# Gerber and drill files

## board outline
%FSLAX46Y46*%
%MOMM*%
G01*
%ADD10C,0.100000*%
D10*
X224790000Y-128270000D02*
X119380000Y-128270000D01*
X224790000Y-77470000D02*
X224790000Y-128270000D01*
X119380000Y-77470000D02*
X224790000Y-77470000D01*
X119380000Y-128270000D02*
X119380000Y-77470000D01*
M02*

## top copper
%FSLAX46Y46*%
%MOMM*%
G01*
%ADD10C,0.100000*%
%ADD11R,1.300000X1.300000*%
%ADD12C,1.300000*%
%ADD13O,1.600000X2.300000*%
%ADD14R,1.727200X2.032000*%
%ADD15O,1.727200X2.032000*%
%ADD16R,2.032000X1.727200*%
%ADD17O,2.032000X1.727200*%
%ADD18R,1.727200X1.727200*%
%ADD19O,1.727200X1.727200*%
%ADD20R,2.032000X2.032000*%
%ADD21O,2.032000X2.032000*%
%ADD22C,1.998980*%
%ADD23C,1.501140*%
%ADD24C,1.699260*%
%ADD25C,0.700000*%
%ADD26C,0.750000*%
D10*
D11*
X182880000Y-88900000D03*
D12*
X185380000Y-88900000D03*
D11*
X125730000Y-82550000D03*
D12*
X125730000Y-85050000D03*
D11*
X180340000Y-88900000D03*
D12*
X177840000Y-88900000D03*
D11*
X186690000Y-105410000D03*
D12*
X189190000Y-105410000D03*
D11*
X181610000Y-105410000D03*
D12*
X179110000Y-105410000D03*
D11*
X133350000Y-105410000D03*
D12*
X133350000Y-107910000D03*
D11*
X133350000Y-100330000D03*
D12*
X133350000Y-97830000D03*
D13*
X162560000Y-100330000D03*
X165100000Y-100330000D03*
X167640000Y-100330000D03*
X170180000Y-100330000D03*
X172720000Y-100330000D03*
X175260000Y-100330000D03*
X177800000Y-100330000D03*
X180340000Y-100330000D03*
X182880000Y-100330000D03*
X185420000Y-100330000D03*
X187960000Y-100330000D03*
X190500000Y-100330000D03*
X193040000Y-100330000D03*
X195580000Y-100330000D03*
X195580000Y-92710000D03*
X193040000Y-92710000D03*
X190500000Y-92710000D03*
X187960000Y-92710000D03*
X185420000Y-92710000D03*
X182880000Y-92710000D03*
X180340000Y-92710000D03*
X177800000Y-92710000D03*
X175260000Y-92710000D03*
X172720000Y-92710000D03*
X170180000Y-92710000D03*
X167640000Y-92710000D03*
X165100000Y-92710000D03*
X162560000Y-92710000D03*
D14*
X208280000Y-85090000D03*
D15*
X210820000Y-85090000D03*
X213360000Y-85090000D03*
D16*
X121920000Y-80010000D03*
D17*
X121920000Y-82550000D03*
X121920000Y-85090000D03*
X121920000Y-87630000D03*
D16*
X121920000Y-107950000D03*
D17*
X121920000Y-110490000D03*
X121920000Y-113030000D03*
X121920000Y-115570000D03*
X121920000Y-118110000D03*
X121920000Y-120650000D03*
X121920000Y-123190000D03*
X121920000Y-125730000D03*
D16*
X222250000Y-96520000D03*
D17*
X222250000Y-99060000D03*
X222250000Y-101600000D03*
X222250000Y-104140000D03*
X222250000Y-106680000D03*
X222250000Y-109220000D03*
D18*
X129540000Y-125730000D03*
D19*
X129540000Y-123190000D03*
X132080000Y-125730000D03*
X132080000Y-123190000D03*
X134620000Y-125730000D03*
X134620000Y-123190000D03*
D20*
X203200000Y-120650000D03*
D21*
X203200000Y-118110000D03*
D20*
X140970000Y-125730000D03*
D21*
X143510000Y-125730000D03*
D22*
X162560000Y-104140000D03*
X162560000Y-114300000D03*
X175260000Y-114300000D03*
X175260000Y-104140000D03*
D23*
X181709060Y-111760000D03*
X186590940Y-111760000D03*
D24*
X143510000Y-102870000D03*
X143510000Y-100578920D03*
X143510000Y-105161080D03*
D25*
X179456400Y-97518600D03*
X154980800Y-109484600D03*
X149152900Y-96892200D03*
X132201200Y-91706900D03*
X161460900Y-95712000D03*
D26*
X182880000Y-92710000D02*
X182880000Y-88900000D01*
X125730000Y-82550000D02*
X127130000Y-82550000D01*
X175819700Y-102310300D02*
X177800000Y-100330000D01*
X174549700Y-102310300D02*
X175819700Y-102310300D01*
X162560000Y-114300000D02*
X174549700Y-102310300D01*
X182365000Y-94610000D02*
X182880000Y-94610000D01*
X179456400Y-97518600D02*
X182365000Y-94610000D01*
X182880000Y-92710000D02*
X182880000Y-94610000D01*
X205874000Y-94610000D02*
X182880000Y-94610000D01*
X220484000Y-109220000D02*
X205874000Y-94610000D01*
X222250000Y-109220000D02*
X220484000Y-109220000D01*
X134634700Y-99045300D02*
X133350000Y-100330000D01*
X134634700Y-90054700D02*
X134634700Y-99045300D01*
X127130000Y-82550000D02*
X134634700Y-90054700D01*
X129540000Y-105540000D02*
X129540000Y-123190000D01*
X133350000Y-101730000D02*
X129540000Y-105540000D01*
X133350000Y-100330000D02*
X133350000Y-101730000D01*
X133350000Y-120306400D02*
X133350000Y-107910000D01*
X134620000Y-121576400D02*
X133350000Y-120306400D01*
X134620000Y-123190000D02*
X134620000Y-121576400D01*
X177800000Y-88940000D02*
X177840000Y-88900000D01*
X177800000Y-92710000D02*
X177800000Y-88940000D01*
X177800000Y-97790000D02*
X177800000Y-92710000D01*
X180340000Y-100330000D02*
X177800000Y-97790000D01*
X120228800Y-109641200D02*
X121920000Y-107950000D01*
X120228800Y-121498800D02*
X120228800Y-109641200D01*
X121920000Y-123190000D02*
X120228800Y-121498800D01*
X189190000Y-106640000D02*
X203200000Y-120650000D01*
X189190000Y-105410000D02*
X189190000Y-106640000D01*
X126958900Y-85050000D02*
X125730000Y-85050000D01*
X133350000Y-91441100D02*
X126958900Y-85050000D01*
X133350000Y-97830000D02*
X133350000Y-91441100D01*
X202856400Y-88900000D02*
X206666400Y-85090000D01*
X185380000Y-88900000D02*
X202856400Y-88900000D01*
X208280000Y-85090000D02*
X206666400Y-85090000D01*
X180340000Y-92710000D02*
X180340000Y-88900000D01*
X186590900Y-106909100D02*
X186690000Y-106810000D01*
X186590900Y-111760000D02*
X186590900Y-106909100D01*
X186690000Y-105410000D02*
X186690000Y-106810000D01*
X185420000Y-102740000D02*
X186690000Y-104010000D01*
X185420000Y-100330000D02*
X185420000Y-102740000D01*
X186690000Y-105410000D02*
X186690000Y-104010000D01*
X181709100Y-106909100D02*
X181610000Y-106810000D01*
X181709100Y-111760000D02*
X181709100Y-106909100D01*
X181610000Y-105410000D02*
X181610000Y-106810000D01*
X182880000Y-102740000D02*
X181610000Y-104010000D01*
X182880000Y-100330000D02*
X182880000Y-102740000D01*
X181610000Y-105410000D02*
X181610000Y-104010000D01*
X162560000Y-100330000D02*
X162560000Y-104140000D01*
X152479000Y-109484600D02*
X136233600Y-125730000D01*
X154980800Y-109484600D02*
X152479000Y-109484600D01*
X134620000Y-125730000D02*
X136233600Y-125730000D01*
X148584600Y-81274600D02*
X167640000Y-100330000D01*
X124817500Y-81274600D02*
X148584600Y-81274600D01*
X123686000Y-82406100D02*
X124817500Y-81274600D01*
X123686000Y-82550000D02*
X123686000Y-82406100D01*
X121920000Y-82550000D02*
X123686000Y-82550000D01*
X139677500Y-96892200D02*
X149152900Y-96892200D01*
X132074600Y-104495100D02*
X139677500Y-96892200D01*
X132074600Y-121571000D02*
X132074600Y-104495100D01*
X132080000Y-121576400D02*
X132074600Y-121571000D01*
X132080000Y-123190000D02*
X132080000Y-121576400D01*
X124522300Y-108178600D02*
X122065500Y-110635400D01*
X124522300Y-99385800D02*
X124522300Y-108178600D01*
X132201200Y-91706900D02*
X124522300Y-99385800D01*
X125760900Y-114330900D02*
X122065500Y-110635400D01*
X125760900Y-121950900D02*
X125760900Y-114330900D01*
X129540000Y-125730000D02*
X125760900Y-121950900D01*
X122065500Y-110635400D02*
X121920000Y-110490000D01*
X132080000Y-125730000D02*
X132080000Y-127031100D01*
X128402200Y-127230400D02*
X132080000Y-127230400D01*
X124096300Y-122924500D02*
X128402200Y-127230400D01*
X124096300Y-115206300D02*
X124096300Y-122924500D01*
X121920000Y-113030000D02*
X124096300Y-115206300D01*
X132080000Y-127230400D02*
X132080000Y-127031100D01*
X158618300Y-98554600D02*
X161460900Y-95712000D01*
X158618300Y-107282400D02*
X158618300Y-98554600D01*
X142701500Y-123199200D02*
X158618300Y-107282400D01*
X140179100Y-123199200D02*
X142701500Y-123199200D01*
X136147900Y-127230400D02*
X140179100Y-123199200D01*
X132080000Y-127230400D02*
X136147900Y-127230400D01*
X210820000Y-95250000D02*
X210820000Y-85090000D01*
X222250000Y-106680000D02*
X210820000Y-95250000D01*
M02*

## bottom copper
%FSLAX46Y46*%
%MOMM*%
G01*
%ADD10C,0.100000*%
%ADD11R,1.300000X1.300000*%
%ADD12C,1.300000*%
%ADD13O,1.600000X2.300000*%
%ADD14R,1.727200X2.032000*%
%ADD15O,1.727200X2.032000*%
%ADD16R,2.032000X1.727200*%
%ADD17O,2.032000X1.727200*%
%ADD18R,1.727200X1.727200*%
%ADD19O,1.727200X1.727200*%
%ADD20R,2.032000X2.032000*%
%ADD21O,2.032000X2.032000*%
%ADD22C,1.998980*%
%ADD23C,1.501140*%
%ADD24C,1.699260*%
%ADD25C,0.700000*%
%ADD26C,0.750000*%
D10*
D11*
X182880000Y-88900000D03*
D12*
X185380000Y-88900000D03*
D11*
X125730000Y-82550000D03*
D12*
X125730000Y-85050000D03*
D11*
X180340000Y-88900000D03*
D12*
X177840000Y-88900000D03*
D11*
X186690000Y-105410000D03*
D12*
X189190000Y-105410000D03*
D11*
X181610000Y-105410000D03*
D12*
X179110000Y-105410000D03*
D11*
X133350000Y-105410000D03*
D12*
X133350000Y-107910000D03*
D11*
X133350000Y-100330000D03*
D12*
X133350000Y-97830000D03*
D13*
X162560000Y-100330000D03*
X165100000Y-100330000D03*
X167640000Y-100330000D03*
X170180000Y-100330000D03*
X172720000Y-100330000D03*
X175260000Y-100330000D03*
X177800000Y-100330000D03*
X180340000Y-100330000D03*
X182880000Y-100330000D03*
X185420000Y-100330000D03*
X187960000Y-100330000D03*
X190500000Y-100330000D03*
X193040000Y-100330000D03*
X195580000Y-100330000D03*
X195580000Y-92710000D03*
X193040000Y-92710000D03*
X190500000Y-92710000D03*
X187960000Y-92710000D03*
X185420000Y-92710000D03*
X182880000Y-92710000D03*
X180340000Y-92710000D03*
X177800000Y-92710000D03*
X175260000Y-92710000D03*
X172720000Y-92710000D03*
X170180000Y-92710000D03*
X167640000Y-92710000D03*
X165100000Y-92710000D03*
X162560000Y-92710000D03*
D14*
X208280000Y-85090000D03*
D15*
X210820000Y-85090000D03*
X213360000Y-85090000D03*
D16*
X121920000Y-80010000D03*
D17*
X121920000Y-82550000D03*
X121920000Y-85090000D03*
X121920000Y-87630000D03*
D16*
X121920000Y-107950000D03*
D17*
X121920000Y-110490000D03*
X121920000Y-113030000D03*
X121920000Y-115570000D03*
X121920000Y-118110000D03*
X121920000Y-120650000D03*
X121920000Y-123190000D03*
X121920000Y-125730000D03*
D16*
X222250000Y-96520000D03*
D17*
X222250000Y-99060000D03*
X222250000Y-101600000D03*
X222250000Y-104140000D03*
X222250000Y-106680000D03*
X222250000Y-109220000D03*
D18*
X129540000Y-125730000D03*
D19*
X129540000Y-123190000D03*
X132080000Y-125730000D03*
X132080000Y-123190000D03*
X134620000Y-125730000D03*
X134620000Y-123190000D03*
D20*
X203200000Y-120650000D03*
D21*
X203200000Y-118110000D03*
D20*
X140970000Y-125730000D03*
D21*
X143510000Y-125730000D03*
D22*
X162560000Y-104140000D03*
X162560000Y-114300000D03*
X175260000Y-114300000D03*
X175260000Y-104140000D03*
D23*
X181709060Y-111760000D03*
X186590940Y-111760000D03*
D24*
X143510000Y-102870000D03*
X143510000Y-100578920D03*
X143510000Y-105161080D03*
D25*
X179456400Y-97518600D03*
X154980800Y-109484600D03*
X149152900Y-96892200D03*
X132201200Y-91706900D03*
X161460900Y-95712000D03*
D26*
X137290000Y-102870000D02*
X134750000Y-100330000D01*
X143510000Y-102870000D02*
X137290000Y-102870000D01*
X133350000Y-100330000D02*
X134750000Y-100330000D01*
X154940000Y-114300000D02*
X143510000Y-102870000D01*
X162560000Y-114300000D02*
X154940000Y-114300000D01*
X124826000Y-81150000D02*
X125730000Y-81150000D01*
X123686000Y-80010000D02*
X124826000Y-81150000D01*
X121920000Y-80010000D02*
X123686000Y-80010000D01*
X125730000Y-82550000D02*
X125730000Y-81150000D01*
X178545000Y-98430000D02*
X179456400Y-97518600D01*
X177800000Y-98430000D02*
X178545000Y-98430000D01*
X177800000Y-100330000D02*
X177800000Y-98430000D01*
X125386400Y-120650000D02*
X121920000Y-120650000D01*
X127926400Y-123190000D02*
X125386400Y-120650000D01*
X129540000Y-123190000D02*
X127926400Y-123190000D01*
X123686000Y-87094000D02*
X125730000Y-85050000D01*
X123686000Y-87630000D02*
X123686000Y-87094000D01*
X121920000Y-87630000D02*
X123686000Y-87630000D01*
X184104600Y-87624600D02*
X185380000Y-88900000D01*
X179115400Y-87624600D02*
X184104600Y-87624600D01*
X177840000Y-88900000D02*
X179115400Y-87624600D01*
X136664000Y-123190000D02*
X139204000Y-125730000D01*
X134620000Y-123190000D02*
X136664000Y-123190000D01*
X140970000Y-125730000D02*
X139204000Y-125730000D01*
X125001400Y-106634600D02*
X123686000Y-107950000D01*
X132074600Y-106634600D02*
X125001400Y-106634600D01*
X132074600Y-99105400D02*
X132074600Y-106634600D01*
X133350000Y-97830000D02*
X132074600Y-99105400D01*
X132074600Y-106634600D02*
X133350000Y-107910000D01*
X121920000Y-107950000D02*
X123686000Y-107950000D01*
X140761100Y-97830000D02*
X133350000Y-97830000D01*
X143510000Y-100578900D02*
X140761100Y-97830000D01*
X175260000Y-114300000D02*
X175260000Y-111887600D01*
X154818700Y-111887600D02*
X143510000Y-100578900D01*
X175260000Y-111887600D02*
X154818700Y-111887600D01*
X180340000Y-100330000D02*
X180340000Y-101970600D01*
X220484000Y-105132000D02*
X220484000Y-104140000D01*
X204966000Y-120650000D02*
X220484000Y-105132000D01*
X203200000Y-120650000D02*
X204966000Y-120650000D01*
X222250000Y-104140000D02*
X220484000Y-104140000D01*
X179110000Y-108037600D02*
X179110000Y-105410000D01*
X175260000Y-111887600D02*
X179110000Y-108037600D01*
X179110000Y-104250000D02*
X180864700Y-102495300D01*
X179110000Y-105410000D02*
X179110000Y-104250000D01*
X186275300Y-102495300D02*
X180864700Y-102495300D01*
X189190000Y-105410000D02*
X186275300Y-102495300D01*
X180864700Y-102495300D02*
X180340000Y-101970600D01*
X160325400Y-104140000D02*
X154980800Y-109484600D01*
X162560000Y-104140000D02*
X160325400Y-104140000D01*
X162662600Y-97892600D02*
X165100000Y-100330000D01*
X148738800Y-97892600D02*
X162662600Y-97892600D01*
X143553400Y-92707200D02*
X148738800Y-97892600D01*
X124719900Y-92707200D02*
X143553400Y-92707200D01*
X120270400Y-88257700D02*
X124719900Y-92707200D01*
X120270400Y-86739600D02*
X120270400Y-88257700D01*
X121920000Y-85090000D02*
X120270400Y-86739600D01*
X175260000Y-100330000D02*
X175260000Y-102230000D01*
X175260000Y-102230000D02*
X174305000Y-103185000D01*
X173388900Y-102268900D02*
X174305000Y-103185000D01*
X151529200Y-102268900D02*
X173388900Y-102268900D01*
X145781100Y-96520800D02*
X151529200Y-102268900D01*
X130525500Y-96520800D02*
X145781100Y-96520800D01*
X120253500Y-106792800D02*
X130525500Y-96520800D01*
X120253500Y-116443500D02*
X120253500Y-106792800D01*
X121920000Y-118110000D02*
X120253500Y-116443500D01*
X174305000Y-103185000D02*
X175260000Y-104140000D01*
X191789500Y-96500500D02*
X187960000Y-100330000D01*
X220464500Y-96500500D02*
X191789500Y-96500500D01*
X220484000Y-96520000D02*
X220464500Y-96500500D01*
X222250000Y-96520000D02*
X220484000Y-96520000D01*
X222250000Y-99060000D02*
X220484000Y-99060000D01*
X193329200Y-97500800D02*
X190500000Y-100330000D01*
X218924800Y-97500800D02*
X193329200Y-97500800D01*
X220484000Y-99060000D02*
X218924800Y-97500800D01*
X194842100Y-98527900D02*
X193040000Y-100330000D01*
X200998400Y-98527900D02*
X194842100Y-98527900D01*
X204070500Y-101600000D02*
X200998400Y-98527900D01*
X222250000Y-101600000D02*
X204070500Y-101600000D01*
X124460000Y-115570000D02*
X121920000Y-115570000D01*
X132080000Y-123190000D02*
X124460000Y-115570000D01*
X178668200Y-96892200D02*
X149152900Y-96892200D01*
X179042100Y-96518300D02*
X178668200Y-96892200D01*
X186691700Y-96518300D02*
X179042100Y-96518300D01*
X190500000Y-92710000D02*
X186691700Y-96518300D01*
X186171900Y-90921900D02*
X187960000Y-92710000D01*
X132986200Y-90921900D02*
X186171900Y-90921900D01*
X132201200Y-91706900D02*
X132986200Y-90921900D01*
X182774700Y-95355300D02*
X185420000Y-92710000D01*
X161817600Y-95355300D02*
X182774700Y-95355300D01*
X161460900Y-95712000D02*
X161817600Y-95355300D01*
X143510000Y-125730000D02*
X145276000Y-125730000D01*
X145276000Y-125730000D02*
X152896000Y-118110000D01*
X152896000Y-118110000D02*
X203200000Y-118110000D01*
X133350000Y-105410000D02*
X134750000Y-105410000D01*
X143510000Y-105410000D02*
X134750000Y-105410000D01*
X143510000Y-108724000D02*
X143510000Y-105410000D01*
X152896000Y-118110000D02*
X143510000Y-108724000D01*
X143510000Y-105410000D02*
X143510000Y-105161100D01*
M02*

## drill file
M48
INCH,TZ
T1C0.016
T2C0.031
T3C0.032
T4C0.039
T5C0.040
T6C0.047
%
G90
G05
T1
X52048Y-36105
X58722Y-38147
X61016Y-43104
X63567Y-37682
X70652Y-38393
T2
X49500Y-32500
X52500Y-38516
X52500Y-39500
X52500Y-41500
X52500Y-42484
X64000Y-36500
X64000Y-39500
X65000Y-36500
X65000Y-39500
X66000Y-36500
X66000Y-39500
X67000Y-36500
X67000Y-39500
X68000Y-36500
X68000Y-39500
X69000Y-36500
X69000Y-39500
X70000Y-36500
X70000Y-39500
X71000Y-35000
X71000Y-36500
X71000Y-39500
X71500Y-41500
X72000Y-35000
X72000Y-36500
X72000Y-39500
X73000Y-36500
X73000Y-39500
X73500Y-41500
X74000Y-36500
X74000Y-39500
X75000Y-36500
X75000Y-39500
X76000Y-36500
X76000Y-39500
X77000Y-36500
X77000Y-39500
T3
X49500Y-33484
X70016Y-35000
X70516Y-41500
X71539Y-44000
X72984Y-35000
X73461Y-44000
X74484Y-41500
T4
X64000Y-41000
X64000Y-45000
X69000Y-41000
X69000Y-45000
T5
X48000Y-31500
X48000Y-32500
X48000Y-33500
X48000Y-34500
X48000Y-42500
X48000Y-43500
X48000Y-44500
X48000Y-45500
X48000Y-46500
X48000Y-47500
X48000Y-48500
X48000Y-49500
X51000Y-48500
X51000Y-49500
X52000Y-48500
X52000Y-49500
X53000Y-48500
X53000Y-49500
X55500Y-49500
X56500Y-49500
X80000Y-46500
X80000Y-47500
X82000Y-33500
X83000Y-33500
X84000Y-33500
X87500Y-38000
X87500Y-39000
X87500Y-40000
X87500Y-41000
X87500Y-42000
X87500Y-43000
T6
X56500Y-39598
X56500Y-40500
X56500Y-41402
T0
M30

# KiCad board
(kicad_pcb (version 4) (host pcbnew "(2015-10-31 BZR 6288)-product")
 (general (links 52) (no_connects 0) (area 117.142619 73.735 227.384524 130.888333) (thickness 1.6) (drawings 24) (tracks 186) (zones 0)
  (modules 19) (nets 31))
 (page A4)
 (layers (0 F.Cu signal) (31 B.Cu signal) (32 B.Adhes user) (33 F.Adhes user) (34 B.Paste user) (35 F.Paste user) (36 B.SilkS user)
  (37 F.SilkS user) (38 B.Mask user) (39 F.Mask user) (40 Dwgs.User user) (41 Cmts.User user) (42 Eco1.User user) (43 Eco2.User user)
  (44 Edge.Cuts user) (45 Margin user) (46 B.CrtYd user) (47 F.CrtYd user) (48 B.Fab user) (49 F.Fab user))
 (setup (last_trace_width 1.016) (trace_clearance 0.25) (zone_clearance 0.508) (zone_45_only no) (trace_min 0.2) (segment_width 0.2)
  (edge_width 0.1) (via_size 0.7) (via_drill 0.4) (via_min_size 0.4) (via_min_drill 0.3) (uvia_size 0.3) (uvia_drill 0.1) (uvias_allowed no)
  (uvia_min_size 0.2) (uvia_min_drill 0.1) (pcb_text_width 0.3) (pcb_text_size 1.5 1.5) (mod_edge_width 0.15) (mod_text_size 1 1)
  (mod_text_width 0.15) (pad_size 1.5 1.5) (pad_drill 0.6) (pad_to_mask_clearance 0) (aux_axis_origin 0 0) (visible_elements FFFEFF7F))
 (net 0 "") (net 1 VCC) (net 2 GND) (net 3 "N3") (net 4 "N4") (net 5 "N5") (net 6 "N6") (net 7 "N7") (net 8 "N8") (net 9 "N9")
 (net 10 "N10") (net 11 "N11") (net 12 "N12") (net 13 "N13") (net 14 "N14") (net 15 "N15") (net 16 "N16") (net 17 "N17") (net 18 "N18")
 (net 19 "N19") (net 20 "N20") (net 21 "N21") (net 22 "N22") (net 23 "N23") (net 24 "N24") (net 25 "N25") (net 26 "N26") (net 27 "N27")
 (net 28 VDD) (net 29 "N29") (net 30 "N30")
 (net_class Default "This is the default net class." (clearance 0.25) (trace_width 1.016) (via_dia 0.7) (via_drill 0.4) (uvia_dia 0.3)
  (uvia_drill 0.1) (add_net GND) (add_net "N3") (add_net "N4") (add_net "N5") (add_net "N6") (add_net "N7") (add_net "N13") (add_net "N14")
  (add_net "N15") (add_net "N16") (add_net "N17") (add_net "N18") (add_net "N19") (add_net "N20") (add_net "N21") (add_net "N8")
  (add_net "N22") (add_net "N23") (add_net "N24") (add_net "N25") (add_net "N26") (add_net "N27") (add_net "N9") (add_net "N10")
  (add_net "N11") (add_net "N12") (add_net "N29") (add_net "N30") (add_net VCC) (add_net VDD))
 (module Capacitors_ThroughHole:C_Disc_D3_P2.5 (layer F.Cu) (at 182.88 88.9)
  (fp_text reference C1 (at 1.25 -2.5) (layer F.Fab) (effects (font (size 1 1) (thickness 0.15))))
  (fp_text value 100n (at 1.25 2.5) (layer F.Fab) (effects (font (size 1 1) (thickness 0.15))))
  (pad 1 thru_hole rect (at 0 0) (size 1.3 1.3) (drill 0.8) (layers *.Cu *.Mask F.SilkS) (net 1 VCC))
  (pad 2 thru_hole circle (at 2.5 0) (size 1.3 1.3) (drill 0.8001) (layers *.Cu *.Mask F.SilkS) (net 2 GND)))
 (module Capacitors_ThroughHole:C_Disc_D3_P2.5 (layer F.Cu) (at 125.73 82.55 270)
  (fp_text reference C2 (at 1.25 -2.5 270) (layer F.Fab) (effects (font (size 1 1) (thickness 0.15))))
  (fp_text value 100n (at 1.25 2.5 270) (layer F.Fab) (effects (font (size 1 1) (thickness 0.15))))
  (pad 1 thru_hole rect (at 0 0 270) (size 1.3 1.3) (drill 0.8) (layers *.Cu *.Mask F.SilkS) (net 1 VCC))
  (pad 2 thru_hole circle (at 2.5 0 270) (size 1.3 1.3) (drill 0.8001) (layers *.Cu *.Mask F.SilkS) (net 2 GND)))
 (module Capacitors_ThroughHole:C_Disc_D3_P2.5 (layer F.Cu) (at 180.34 88.9 180)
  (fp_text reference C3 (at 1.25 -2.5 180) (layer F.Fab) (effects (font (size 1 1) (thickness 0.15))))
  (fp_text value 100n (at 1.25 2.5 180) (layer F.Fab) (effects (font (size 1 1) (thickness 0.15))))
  (pad 1 thru_hole rect (at 0 0 180) (size 1.3 1.3) (drill 0.8) (layers *.Cu *.Mask F.SilkS) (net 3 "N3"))
  (pad 2 thru_hole circle (at 2.5 0 180) (size 1.3 1.3) (drill 0.8001) (layers *.Cu *.Mask F.SilkS) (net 2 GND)))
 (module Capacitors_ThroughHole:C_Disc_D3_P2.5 (layer F.Cu) (at 186.69 105.41)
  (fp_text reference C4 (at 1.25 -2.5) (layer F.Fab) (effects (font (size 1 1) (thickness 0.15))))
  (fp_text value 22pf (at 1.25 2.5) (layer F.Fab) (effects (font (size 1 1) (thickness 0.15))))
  (pad 1 thru_hole rect (at 0 0) (size 1.3 1.3) (drill 0.8) (layers *.Cu *.Mask F.SilkS) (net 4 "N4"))
  (pad 2 thru_hole circle (at 2.5 0) (size 1.3 1.3) (drill 0.8001) (layers *.Cu *.Mask F.SilkS) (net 2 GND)))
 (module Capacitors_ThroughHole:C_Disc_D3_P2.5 (layer F.Cu) (at 181.61 105.41 180)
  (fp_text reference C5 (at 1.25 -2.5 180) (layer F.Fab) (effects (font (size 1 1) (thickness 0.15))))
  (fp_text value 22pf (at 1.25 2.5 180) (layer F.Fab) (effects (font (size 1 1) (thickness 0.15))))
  (pad 1 thru_hole rect (at 0 0 180) (size 1.3 1.3) (drill 0.8) (layers *.Cu *.Mask F.SilkS) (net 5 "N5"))
  (pad 2 thru_hole circle (at 2.5 0 180) (size 1.3 1.3) (drill 0.8001) (layers *.Cu *.Mask F.SilkS) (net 2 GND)))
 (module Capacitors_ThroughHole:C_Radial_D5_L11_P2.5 (layer F.Cu) (at 133.35 105.41 270)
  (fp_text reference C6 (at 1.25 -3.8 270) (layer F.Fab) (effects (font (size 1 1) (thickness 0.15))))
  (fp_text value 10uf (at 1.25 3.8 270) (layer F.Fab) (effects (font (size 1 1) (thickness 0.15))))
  (pad 1 thru_hole rect (at 0 0 270) (size 1.3 1.3) (drill 0.8) (layers *.Cu *.Mask F.SilkS) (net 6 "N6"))
  (pad 2 thru_hole circle (at 2.5 0 270) (size 1.3 1.3) (drill 0.8) (layers *.Cu *.Mask F.SilkS) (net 2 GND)))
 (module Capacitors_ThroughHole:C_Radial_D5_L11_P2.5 (layer F.Cu) (at 133.35 100.33 90)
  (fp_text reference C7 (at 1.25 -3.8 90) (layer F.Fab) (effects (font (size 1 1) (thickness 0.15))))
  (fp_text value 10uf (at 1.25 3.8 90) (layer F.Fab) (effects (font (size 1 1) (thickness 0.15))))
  (pad 1 thru_hole rect (at 0 0 90) (size 1.3 1.3) (drill 0.8) (layers *.Cu *.Mask F.SilkS) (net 1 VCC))
  (pad 2 thru_hole circle (at 2.5 0 90) (size 1.3 1.3) (drill 0.8) (layers *.Cu *.Mask F.SilkS) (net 2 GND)))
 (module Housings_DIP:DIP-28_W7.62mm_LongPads (layer F.Cu) (at 162.56 100.33 90)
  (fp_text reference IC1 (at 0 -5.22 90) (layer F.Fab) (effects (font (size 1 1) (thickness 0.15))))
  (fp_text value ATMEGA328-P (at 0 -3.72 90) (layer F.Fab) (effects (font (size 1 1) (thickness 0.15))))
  (pad 1 thru_hole oval (at 0 0 90) (size 2.3 1.6) (drill 0.8) (layers *.Cu *.Mask F.SilkS) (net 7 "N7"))
  (pad 2 thru_hole oval (at 0 2.54 90) (size 2.3 1.6) (drill 0.8) (layers *.Cu *.Mask F.SilkS) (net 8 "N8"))
  (pad 3 thru_hole oval (at 0 5.08 90) (size 2.3 1.6) (drill 0.8) (layers *.Cu *.Mask F.SilkS) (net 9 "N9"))
  (pad 4 thru_hole oval (at 0 7.62 90) (size 2.3 1.6) (drill 0.8) (layers *.Cu *.Mask F.SilkS) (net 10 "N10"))
  (pad 5 thru_hole oval (at 0 10.16 90) (size 2.3 1.6) (drill 0.8) (layers *.Cu *.Mask F.SilkS) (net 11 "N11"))
  (pad 6 thru_hole oval (at 0 12.7 90) (size 2.3 1.6) (drill 0.8) (layers *.Cu *.Mask F.SilkS) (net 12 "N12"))
  (pad 7 thru_hole oval (at 0 15.24 90) (size 2.3 1.6) (drill 0.8) (layers *.Cu *.Mask F.SilkS) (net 1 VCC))
  (pad 8 thru_hole oval (at 0 17.78 90) (size 2.3 1.6) (drill 0.8) (layers *.Cu *.Mask F.SilkS) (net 2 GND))
  (pad 9 thru_hole oval (at 0 20.32 90) (size 2.3 1.6) (drill 0.8) (layers *.Cu *.Mask F.SilkS) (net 5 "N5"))
  (pad 10 thru_hole oval (at 0 22.86 90) (size 2.3 1.6) (drill 0.8) (layers *.Cu *.Mask F.SilkS) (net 4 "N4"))
  (pad 11 thru_hole oval (at 0 25.4 90) (size 2.3 1.6) (drill 0.8) (layers *.Cu *.Mask F.SilkS) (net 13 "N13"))
  (pad 12 thru_hole oval (at 0 27.94 90) (size 2.3 1.6) (drill 0.8) (layers *.Cu *.Mask F.SilkS) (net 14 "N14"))
  (pad 13 thru_hole oval (at 0 30.48 90) (size 2.3 1.6) (drill 0.8) (layers *.Cu *.Mask F.SilkS) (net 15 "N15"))
  (pad 14 thru_hole oval (at 0 33.02 90) (size 2.3 1.6) (drill 0.8) (layers *.Cu *.Mask F.SilkS) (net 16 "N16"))
  (pad 15 thru_hole oval (at 7.62 33.02 90) (size 2.3 1.6) (drill 0.8) (layers *.Cu *.Mask F.SilkS) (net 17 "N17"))
  (pad 16 thru_hole oval (at 7.62 30.48 90) (size 2.3 1.6) (drill 0.8) (layers *.Cu *.Mask F.SilkS) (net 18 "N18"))
  (pad 17 thru_hole oval (at 7.62 27.94 90) (size 2.3 1.6) (drill 0.8) (layers *.Cu *.Mask F.SilkS) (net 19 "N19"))
  (pad 18 thru_hole oval (at 7.62 25.4 90) (size 2.3 1.6) (drill 0.8) (layers *.Cu *.Mask F.SilkS) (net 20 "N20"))
  (pad 19 thru_hole oval (at 7.62 22.86 90) (size 2.3 1.6) (drill 0.8) (layers *.Cu *.Mask F.SilkS) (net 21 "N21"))
  (pad 20 thru_hole oval (at 7.62 20.32 90) (size 2.3 1.6) (drill 0.8) (layers *.Cu *.Mask F.SilkS) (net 1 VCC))
  (pad 21 thru_hole oval (at 7.62 17.78 90) (size 2.3 1.6) (drill 0.8) (layers *.Cu *.Mask F.SilkS) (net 3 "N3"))
  (pad 22 thru_hole oval (at 7.62 15.24 90) (size 2.3 1.6) (drill 0.8) (layers *.Cu *.Mask F.SilkS) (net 2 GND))
  (pad 23 thru_hole oval (at 7.62 12.7 90) (size 2.3 1.6) (drill 0.8) (layers *.Cu *.Mask F.SilkS) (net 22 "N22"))
  (pad 24 thru_hole oval (at 7.62 10.16 90) (size 2.3 1.6) (drill 0.8) (layers *.Cu *.Mask F.SilkS) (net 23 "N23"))
  (pad 25 thru_hole oval (at 7.62 7.62 90) (size 2.3 1.6) (drill 0.8) (layers *.Cu *.Mask F.SilkS) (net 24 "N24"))
  (pad 26 thru_hole oval (at 7.62 5.08 90) (size 2.3 1.6) (drill 0.8) (layers *.Cu *.Mask F.SilkS) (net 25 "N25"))
  (pad 27 thru_hole oval (at 7.62 2.54 90) (size 2.3 1.6) (drill 0.8) (layers *.Cu *.Mask F.SilkS) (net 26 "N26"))
  (pad 28 thru_hole oval (at 7.62 0 90) (size 2.3 1.6) (drill 0.8) (layers *.Cu *.Mask F.SilkS) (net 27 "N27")))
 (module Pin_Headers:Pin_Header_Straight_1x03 (layer F.Cu) (at 208.28 85.09 90)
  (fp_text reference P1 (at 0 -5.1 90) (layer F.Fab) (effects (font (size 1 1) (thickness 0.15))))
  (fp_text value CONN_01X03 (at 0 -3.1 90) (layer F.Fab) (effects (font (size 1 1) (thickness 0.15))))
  (pad 1 thru_hole rect (at 0 0 90) (size 2.032 1.7272) (drill 1.016) (layers *.Cu *.Mask F.SilkS) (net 2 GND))
  (pad 2 thru_hole oval (at 0 2.54 90) (size 2.032 1.7272) (drill 1.016) (layers *.Cu *.Mask F.SilkS) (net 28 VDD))
  (pad 3 thru_hole oval (at 0 5.08 90) (size 2.032 1.7272) (drill 1.016) (layers *.Cu *.Mask F.SilkS) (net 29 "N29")))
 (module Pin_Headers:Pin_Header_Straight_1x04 (layer F.Cu) (at 121.92 80.01)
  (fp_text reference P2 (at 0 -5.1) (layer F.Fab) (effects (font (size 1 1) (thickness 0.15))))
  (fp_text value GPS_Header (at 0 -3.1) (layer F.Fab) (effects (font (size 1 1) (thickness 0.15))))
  (pad 1 thru_hole rect (at 0 0) (size 2.032 1.7272) (drill 1.016) (layers *.Cu *.Mask F.SilkS) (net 1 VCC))
  (pad 2 thru_hole oval (at 0 2.54) (size 2.032 1.7272) (drill 1.016) (layers *.Cu *.Mask F.SilkS) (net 9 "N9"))
  (pad 3 thru_hole oval (at 0 5.08) (size 2.032 1.7272) (drill 1.016) (layers *.Cu *.Mask F.SilkS) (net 8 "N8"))
  (pad 4 thru_hole oval (at 0 7.62) (size 2.032 1.7272) (drill 1.016) (layers *.Cu *.Mask F.SilkS) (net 2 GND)))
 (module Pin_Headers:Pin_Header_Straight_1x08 (layer F.Cu) (at 121.92 107.95)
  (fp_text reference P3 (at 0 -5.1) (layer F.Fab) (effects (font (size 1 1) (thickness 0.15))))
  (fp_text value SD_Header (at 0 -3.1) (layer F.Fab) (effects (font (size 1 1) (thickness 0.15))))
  (pad 1 thru_hole rect (at 0 0) (size 2.032 1.7272) (drill 1.016) (layers *.Cu *.Mask F.SilkS) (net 2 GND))
  (pad 2 thru_hole oval (at 0 2.54) (size 2.032 1.7272) (drill 1.016) (layers *.Cu *.Mask F.SilkS) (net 20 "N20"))
  (pad 3 thru_hole oval (at 0 5.08) (size 2.032 1.7272) (drill 1.016) (layers *.Cu *.Mask F.SilkS) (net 21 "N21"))
  (pad 4 thru_hole oval (at 0 7.62) (size 2.032 1.7272) (drill 1.016) (layers *.Cu *.Mask F.SilkS) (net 19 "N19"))
  (pad 5 thru_hole oval (at 0 10.16) (size 2.032 1.7272) (drill 1.016) (layers *.Cu *.Mask F.SilkS) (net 12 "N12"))
  (pad 6 thru_hole oval (at 0 12.7) (size 2.032 1.7272) (drill 1.016) (layers *.Cu *.Mask F.SilkS) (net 1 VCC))
  (pad 7 thru_hole oval (at 0 15.24) (size 2.032 1.7272) (drill 1.016) (layers *.Cu *.Mask F.SilkS) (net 2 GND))
  (pad 8 thru_hole oval (at 0 17.78) (size 2.032 1.7272) (drill 1.016) (layers *.Cu *.Mask F.SilkS) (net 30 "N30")))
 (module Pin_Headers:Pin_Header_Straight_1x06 (layer F.Cu) (at 222.25 96.52)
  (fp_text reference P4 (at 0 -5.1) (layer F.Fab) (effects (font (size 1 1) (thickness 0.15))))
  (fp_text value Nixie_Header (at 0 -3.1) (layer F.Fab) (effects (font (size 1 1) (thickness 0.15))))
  (pad 1 thru_hole rect (at 0 0) (size 2.032 1.7272) (drill 1.016) (layers *.Cu *.Mask F.SilkS) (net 13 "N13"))
  (pad 2 thru_hole oval (at 0 2.54) (size 2.032 1.7272) (drill 1.016) (layers *.Cu *.Mask F.SilkS) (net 14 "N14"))
  (pad 3 thru_hole oval (at 0 5.08) (size 2.032 1.7272) (drill 1.016) (layers *.Cu *.Mask F.SilkS) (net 15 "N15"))
  (pad 4 thru_hole oval (at 0 7.62) (size 2.032 1.7272) (drill 1.016) (layers *.Cu *.Mask F.SilkS) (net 2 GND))
  (pad 5 thru_hole oval (at 0 10.16) (size 2.032 1.7272) (drill 1.016) (layers *.Cu *.Mask F.SilkS) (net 28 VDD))
  (pad 6 thru_hole oval (at 0 12.7) (size 2.032 1.7272) (drill 1.016) (layers *.Cu *.Mask F.SilkS) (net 1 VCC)))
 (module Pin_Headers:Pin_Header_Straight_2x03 (layer F.Cu) (at 129.54 125.73 90)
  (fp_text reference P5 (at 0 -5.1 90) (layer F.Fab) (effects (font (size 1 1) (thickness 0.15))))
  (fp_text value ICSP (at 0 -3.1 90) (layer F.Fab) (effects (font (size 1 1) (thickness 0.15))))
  (pad 1 thru_hole rect (at 0 0 90) (size 1.7272 1.7272) (drill 1.016) (layers *.Cu *.Mask F.SilkS) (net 20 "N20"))
  (pad 2 thru_hole oval (at 2.54 0 90) (size 1.7272 1.7272) (drill 1.016) (layers *.Cu *.Mask F.SilkS) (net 1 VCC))
  (pad 3 thru_hole oval (at 0 2.54 90) (size 1.7272 1.7272) (drill 1.016) (layers *.Cu *.Mask F.SilkS) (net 21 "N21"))
  (pad 4 thru_hole oval (at 2.54 2.54 90) (size 1.7272 1.7272) (drill 1.016) (layers *.Cu *.Mask F.SilkS) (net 19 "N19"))
  (pad 5 thru_hole oval (at 0 5.08 90) (size 1.7272 1.7272) (drill 1.016) (layers *.Cu *.Mask F.SilkS) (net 7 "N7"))
  (pad 6 thru_hole oval (at 2.54 5.08 90) (size 1.7272 1.7272) (drill 1.016) (layers *.Cu *.Mask F.SilkS) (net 2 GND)))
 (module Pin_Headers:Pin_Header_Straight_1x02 (layer F.Cu) (at 203.2 120.65 180)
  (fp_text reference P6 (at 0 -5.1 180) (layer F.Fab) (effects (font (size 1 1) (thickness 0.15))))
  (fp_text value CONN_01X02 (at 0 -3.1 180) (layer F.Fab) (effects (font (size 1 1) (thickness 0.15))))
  (pad 1 thru_hole rect (at 0 0 180) (size 2.032 2.032) (drill 1.016) (layers *.Cu *.Mask F.SilkS) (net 2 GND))
  (pad 2 thru_hole oval (at 0 2.54 180) (size 2.032 2.032) (drill 1.016) (layers *.Cu *.Mask F.SilkS) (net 6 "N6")))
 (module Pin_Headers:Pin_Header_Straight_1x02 (layer F.Cu) (at 140.97 125.73 90)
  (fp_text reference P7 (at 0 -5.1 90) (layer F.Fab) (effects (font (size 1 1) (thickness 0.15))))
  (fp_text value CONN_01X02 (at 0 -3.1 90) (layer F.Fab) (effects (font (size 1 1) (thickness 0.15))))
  (pad 1 thru_hole rect (at 0 0 90) (size 2.032 2.032) (drill 1.016) (layers *.Cu *.Mask F.SilkS) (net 2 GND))
  (pad 2 thru_hole oval (at 0 2.54 90) (size 2.032 2.032) (drill 1.016) (layers *.Cu *.Mask F.SilkS) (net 6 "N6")))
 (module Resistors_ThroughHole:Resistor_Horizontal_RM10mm (layer F.Cu) (at 162.56 104.14 270)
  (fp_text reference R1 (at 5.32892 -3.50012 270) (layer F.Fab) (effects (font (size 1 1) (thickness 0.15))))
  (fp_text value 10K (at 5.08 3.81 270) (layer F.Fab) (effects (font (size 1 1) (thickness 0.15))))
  (pad 1 thru_hole circle (at 0 0 270) (size 1.99898 1.99898) (drill 1.00076) (layers *.Cu *.SilkS *.Mask) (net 7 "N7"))
  (pad 2 thru_hole circle (at 10.16 0 270) (size 1.99898 1.99898) (drill 1.00076) (layers *.Cu *.SilkS *.Mask) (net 1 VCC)))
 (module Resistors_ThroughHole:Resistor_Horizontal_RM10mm (layer F.Cu) (at 175.26 114.3 90)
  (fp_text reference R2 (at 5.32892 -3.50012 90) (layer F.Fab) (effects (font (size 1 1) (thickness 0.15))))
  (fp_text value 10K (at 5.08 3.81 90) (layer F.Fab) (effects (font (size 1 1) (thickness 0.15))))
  (pad 1 thru_hole circle (at 0 0 90) (size 1.99898 1.99898) (drill 1.00076) (layers *.Cu *.SilkS *.Mask) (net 2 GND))
  (pad 2 thru_hole circle (at 10.16 0 90) (size 1.99898 1.99898) (drill 1.00076) (layers *.Cu *.SilkS *.Mask) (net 12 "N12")))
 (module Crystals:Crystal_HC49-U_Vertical (layer F.Cu) (at 184.15 111.76)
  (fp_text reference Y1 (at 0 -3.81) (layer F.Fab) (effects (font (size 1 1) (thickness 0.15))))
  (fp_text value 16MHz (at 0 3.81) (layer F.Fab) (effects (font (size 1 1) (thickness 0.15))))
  (pad 1 thru_hole circle (at -2.44094 0) (size 1.50114 1.50114) (drill 0.8001) (layers *.Cu *.Mask F.SilkS) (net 5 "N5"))
  (pad 2 thru_hole circle (at 2.44094 0) (size 1.50114 1.50114) (drill 0.8001) (layers *.Cu *.Mask F.SilkS) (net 4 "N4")))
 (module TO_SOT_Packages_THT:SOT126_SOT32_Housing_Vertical (layer F.Cu) (at 143.51 102.87 270)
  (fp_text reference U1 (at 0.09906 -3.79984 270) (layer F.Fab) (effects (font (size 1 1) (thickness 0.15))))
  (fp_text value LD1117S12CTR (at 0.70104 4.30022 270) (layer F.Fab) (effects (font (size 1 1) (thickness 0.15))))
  (pad 2 thru_hole circle (at 0 0 270) (size 1.69926 1.69926) (drill 1.19888) (layers *.Cu *.Mask F.SilkS) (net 1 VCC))
  (pad 1 thru_hole circle (at -2.29108 0 270) (size 1.69926 1.69926) (drill 1.19888) (layers *.Cu *.Mask F.SilkS) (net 2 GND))
  (pad 3 thru_hole circle (at 2.29108 0 270) (size 1.69926 1.69926) (drill 1.19888) (layers *.Cu *.Mask F.SilkS) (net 6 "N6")))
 (gr_line (start 224.79 128.27) (end 119.38 128.27) (angle 90) (layer Edge.Cuts) (width 0.1))
 (gr_line (start 224.79 77.47) (end 224.79 128.27) (angle 90) (layer Edge.Cuts) (width 0.1))
 (gr_line (start 119.38 77.47) (end 224.79 77.47) (angle 90) (layer Edge.Cuts) (width 0.1))
 (gr_line (start 119.38 128.27) (end 119.38 77.47) (angle 90) (layer Edge.Cuts) (width 0.1))
 (via (at 179.4564 97.5186) (size 0.7) (layers F.Cu B.Cu) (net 1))
 (segment (start 137.29 102.87) (end 134.75 100.33) (width 0.75) (layer B.Cu) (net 1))
 (segment (start 143.51 102.87) (end 137.29 102.87) (width 0.75) (layer B.Cu) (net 1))
 (segment (start 133.35 100.33) (end 134.75 100.33) (width 0.75) (layer B.Cu) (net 1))
 (segment (start 154.94 114.3) (end 143.51 102.87) (width 0.75) (layer B.Cu) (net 1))
 (segment (start 162.56 114.3) (end 154.94 114.3) (width 0.75) (layer B.Cu) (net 1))
 (segment (start 124.826 81.15) (end 125.73 81.15) (width 0.75) (layer B.Cu) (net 1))
 (segment (start 123.686 80.01) (end 124.826 81.15) (width 0.75) (layer B.Cu) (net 1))
 (segment (start 121.92 80.01) (end 123.686 80.01) (width 0.75) (layer B.Cu) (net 1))
 (segment (start 125.73 82.55) (end 125.73 81.15) (width 0.75) (layer B.Cu) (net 1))
 (segment (start 182.88 92.71) (end 182.88 88.9) (width 0.75) (layer F.Cu) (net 1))
 (segment (start 125.73 82.55) (end 127.13 82.55) (width 0.75) (layer F.Cu) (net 1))
 (segment (start 175.8197 102.3103) (end 177.8 100.33) (width 0.75) (layer F.Cu) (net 1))
 (segment (start 174.5497 102.3103) (end 175.8197 102.3103) (width 0.75) (layer F.Cu) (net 1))
 (segment (start 162.56 114.3) (end 174.5497 102.3103) (width 0.75) (layer F.Cu) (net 1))
 (segment (start 178.545 98.43) (end 179.4564 97.5186) (width 0.75) (layer B.Cu) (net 1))
 (segment (start 177.8 98.43) (end 178.545 98.43) (width 0.75) (layer B.Cu) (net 1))
 (segment (start 182.365 94.61) (end 182.88 94.61) (width 0.75) (layer F.Cu) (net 1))
 (segment (start 179.4564 97.5186) (end 182.365 94.61) (width 0.75) (layer F.Cu) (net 1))
 (segment (start 182.88 92.71) (end 182.88 94.61) (width 0.75) (layer F.Cu) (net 1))
 (segment (start 177.8 100.33) (end 177.8 98.43) (width 0.75) (layer B.Cu) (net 1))
 (segment (start 205.874 94.61) (end 182.88 94.61) (width 0.75) (layer F.Cu) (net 1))
 (segment (start 220.484 109.22) (end 205.874 94.61) (width 0.75) (layer F.Cu) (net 1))
 (segment (start 222.25 109.22) (end 220.484 109.22) (width 0.75) (layer F.Cu) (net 1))
 (segment (start 125.3864 120.65) (end 121.92 120.65) (width 0.75) (layer B.Cu) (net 1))
 (segment (start 127.9264 123.19) (end 125.3864 120.65) (width 0.75) (layer B.Cu) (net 1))
 (segment (start 129.54 123.19) (end 127.9264 123.19) (width 0.75) (layer B.Cu) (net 1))
 (segment (start 134.6347 99.0453) (end 133.35 100.33) (width 0.75) (layer F.Cu) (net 1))
 (segment (start 134.6347 90.0547) (end 134.6347 99.0453) (width 0.75) (layer F.Cu) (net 1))
 (segment (start 127.13 82.55) (end 134.6347 90.0547) (width 0.75) (layer F.Cu) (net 1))
 (segment (start 129.54 105.54) (end 129.54 123.19) (width 0.75) (layer F.Cu) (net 1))
 (segment (start 133.35 101.73) (end 129.54 105.54) (width 0.75) (layer F.Cu) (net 1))
 (segment (start 133.35 100.33) (end 133.35 101.73) (width 0.75) (layer F.Cu) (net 1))
 (segment (start 133.35 120.3064) (end 133.35 107.91) (width 0.75) (layer F.Cu) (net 2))
 (segment (start 134.62 121.5764) (end 133.35 120.3064) (width 0.75) (layer F.Cu) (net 2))
 (segment (start 134.62 123.19) (end 134.62 121.5764) (width 0.75) (layer F.Cu) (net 2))
 (segment (start 123.686 87.094) (end 125.73 85.05) (width 0.75) (layer B.Cu) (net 2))
 (segment (start 123.686 87.63) (end 123.686 87.094) (width 0.75) (layer B.Cu) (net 2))
 (segment (start 121.92 87.63) (end 123.686 87.63) (width 0.75) (layer B.Cu) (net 2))
 (segment (start 177.8 88.94) (end 177.84 88.9) (width 0.75) (layer F.Cu) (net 2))
 (segment (start 177.8 92.71) (end 177.8 88.94) (width 0.75) (layer F.Cu) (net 2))
 (segment (start 177.8 97.79) (end 177.8 92.71) (width 0.75) (layer F.Cu) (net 2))
 (segment (start 180.34 100.33) (end 177.8 97.79) (width 0.75) (layer F.Cu) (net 2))
 (segment (start 120.2288 109.6412) (end 121.92 107.95) (width 0.75) (layer F.Cu) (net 2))
 (segment (start 120.2288 121.4988) (end 120.2288 109.6412) (width 0.75) (layer F.Cu) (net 2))
 (segment (start 121.92 123.19) (end 120.2288 121.4988) (width 0.75) (layer F.Cu) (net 2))
 (segment (start 184.1046 87.6246) (end 185.38 88.9) (width 0.75) (layer B.Cu) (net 2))
 (segment (start 179.1154 87.6246) (end 184.1046 87.6246) (width 0.75) (layer B.Cu) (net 2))
 (segment (start 177.84 88.9) (end 179.1154 87.6246) (width 0.75) (layer B.Cu) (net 2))
 (segment (start 136.664 123.19) (end 139.204 125.73) (width 0.75) (layer B.Cu) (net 2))
 (segment (start 134.62 123.19) (end 136.664 123.19) (width 0.75) (layer B.Cu) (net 2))
 (segment (start 140.97 125.73) (end 139.204 125.73) (width 0.75) (layer B.Cu) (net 2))
 (segment (start 189.19 106.64) (end 203.2 120.65) (width 0.75) (layer F.Cu) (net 2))
 (segment (start 189.19 105.41) (end 189.19 106.64) (width 0.75) (layer F.Cu) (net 2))
 (segment (start 126.9589 85.05) (end 125.73 85.05) (width 0.75) (layer F.Cu) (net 2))
 (segment (start 133.35 91.4411) (end 126.9589 85.05) (width 0.75) (layer F.Cu) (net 2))
 (segment (start 133.35 97.83) (end 133.35 91.4411) (width 0.75) (layer F.Cu) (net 2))
 (segment (start 125.0014 106.6346) (end 123.686 107.95) (width 0.75) (layer B.Cu) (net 2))
 (segment (start 132.0746 106.6346) (end 125.0014 106.6346) (width 0.75) (layer B.Cu) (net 2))
 (segment (start 132.0746 99.1054) (end 132.0746 106.6346) (width 0.75) (layer B.Cu) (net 2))
 (segment (start 133.35 97.83) (end 132.0746 99.1054) (width 0.75) (layer B.Cu) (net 2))
 (segment (start 132.0746 106.6346) (end 133.35 107.91) (width 0.75) (layer B.Cu) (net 2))
 (segment (start 121.92 107.95) (end 123.686 107.95) (width 0.75) (layer B.Cu) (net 2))
 (segment (start 140.7611 97.83) (end 133.35 97.83) (width 0.75) (layer B.Cu) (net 2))
 (segment (start 143.51 100.5789) (end 140.7611 97.83) (width 0.75) (layer B.Cu) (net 2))
 (segment (start 175.26 114.3) (end 175.26 111.8876) (width 0.75) (layer B.Cu) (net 2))
 (segment (start 154.8187 111.8876) (end 143.51 100.5789) (width 0.75) (layer B.Cu) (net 2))
 (segment (start 175.26 111.8876) (end 154.8187 111.8876) (width 0.75) (layer B.Cu) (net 2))
 (segment (start 180.34 100.33) (end 180.34 101.9706) (width 0.75) (layer B.Cu) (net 2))
 (segment (start 202.8564 88.9) (end 206.6664 85.09) (width 0.75) (layer F.Cu) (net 2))
 (segment (start 185.38 88.9) (end 202.8564 88.9) (width 0.75) (layer F.Cu) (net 2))
 (segment (start 208.28 85.09) (end 206.6664 85.09) (width 0.75) (layer F.Cu) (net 2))
 (segment (start 220.484 105.132) (end 220.484 104.14) (width 0.75) (layer B.Cu) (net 2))
 (segment (start 204.966 120.65) (end 220.484 105.132) (width 0.75) (layer B.Cu) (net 2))
 (segment (start 203.2 120.65) (end 204.966 120.65) (width 0.75) (layer B.Cu) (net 2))
 (segment (start 222.25 104.14) (end 220.484 104.14) (width 0.75) (layer B.Cu) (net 2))
 (segment (start 179.11 108.0376) (end 179.11 105.41) (width 0.75) (layer B.Cu) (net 2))
 (segment (start 175.26 111.8876) (end 179.11 108.0376) (width 0.75) (layer B.Cu) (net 2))
 (segment (start 179.11 104.25) (end 180.8647 102.4953) (width 0.75) (layer B.Cu) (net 2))
 (segment (start 179.11 105.41) (end 179.11 104.25) (width 0.75) (layer B.Cu) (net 2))
 (segment (start 186.2753 102.4953) (end 180.8647 102.4953) (width 0.75) (layer B.Cu) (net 2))
 (segment (start 189.19 105.41) (end 186.2753 102.4953) (width 0.75) (layer B.Cu) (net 2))
 (segment (start 180.8647 102.4953) (end 180.34 101.9706) (width 0.75) (layer B.Cu) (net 2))
 (segment (start 180.34 92.71) (end 180.34 88.9) (width 0.75) (layer F.Cu) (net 3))
 (segment (start 186.5909 106.9091) (end 186.69 106.81) (width 0.75) (layer F.Cu) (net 4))
 (segment (start 186.5909 111.76) (end 186.5909 106.9091) (width 0.75) (layer F.Cu) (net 4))
 (segment (start 186.69 105.41) (end 186.69 106.81) (width 0.75) (layer F.Cu) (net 4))
 (segment (start 185.42 102.74) (end 186.69 104.01) (width 0.75) (layer F.Cu) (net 4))
 (segment (start 185.42 100.33) (end 185.42 102.74) (width 0.75) (layer F.Cu) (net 4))
 (segment (start 186.69 105.41) (end 186.69 104.01) (width 0.75) (layer F.Cu) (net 4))
 (segment (start 181.7091 106.9091) (end 181.61 106.81) (width 0.75) (layer F.Cu) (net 5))
 (segment (start 181.7091 111.76) (end 181.7091 106.9091) (width 0.75) (layer F.Cu) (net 5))
 (segment (start 181.61 105.41) (end 181.61 106.81) (width 0.75) (layer F.Cu) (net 5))
 (segment (start 182.88 102.74) (end 181.61 104.01) (width 0.75) (layer F.Cu) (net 5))
 (segment (start 182.88 100.33) (end 182.88 102.74) (width 0.75) (layer F.Cu) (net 5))
 (segment (start 181.61 105.41) (end 181.61 104.01) (width 0.75) (layer F.Cu) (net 5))
 (via (at 154.9808 109.4846) (size 0.7) (layers F.Cu B.Cu) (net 7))
 (segment (start 162.56 100.33) (end 162.56 104.14) (width 0.75) (layer F.Cu) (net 7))
 (segment (start 160.3254 104.14) (end 154.9808 109.4846) (width 0.75) (layer B.Cu) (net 7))
 (segment (start 162.56 104.14) (end 160.3254 104.14) (width 0.75) (layer B.Cu) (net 7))
 (segment (start 152.479 109.4846) (end 136.2336 125.73) (width 0.75) (layer F.Cu) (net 7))
 (segment (start 154.9808 109.4846) (end 152.479 109.4846) (width 0.75) (layer F.Cu) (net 7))
 (segment (start 134.62 125.73) (end 136.2336 125.73) (width 0.75) (layer F.Cu) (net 7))
 (segment (start 162.6626 97.8926) (end 165.1 100.33) (width 0.75) (layer B.Cu) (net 8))
 (segment (start 148.7388 97.8926) (end 162.6626 97.8926) (width 0.75) (layer B.Cu) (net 8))
 (segment (start 143.5534 92.7072) (end 148.7388 97.8926) (width 0.75) (layer B.Cu) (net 8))
 (segment (start 124.7199 92.7072) (end 143.5534 92.7072) (width 0.75) (layer B.Cu) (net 8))
 (segment (start 120.2704 88.2577) (end 124.7199 92.7072) (width 0.75) (layer B.Cu) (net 8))
 (segment (start 120.2704 86.7396) (end 120.2704 88.2577) (width 0.75) (layer B.Cu) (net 8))
 (segment (start 121.92 85.09) (end 120.2704 86.7396) (width 0.75) (layer B.Cu) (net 8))
 (segment (start 148.5846 81.2746) (end 167.64 100.33) (width 0.75) (layer F.Cu) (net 9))
 (segment (start 124.8175 81.2746) (end 148.5846 81.2746) (width 0.75) (layer F.Cu) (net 9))
 (segment (start 123.686 82.4061) (end 124.8175 81.2746) (width 0.75) (layer F.Cu) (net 9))
 (segment (start 123.686 82.55) (end 123.686 82.4061) (width 0.75) (layer F.Cu) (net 9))
 (segment (start 121.92 82.55) (end 123.686 82.55) (width 0.75) (layer F.Cu) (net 9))
 (segment (start 175.26 100.33) (end 175.26 102.23) (width 0.75) (layer B.Cu) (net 12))
 (segment (start 175.26 102.23) (end 174.305 103.185) (width 0.75) (layer B.Cu) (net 12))
 (segment (start 173.3889 102.2689) (end 174.305 103.185) (width 0.75) (layer B.Cu) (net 12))
 (segment (start 151.5292 102.2689) (end 173.3889 102.2689) (width 0.75) (layer B.Cu) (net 12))
 (segment (start 145.7811 96.5208) (end 151.5292 102.2689) (width 0.75) (layer B.Cu) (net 12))
 (segment (start 130.5255 96.5208) (end 145.7811 96.5208) (width 0.75) (layer B.Cu) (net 12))
 (segment (start 120.2535 106.7928) (end 130.5255 96.5208) (width 0.75) (layer B.Cu) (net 12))
 (segment (start 120.2535 116.4435) (end 120.2535 106.7928) (width 0.75) (layer B.Cu) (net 12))
 (segment (start 121.92 118.11) (end 120.2535 116.4435) (width 0.75) (layer B.Cu) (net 12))
 (segment (start 174.305 103.185) (end 175.26 104.14) (width 0.75) (layer B.Cu) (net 12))
 (segment (start 191.7895 96.5005) (end 187.96 100.33) (width 0.75) (layer B.Cu) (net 13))
 (segment (start 220.4645 96.5005) (end 191.7895 96.5005) (width 0.75) (layer B.Cu) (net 13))
 (segment (start 220.484 96.52) (end 220.4645 96.5005) (width 0.75) (layer B.Cu) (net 13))
 (segment (start 222.25 96.52) (end 220.484 96.52) (width 0.75) (layer B.Cu) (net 13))
 (segment (start 222.25 99.06) (end 220.484 99.06) (width 0.75) (layer B.Cu) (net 14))
 (segment (start 193.3292 97.5008) (end 190.5 100.33) (width 0.75) (layer B.Cu) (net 14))
 (segment (start 218.9248 97.5008) (end 193.3292 97.5008) (width 0.75) (layer B.Cu) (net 14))
 (segment (start 220.484 99.06) (end 218.9248 97.5008) (width 0.75) (layer B.Cu) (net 14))
 (segment (start 194.8421 98.5279) (end 193.04 100.33) (width 0.75) (layer B.Cu) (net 15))
 (segment (start 200.9984 98.5279) (end 194.8421 98.5279) (width 0.75) (layer B.Cu) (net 15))
 (segment (start 204.0705 101.6) (end 200.9984 98.5279) (width 0.75) (layer B.Cu) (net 15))
 (segment (start 222.25 101.6) (end 204.0705 101.6) (width 0.75) (layer B.Cu) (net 15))
 (via (at 149.1529 96.8922) (size 0.7) (layers F.Cu B.Cu) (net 19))
 (segment (start 139.6775 96.8922) (end 149.1529 96.8922) (width 0.75) (layer F.Cu) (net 19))
 (segment (start 132.0746 104.4951) (end 139.6775 96.8922) (width 0.75) (layer F.Cu) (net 19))
 (segment (start 132.0746 121.571) (end 132.0746 104.4951) (width 0.75) (layer F.Cu) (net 19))
 (segment (start 132.08 121.5764) (end 132.0746 121.571) (width 0.75) (layer F.Cu) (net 19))
 (segment (start 132.08 123.19) (end 132.08 121.5764) (width 0.75) (layer F.Cu) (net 19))
 (segment (start 124.46 115.57) (end 121.92 115.57) (width 0.75) (layer B.Cu) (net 19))
 (segment (start 132.08 123.19) (end 124.46 115.57) (width 0.75) (layer B.Cu) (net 19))
 (segment (start 178.6682 96.8922) (end 149.1529 96.8922) (width 0.75) (layer B.Cu) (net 19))
 (segment (start 179.0421 96.5183) (end 178.6682 96.8922) (width 0.75) (layer B.Cu) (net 19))
 (segment (start 186.6917 96.5183) (end 179.0421 96.5183) (width 0.75) (layer B.Cu) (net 19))
 (segment (start 190.5 92.71) (end 186.6917 96.5183) (width 0.75) (layer B.Cu) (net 19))
 (via (at 132.2012 91.7069) (size 0.7) (layers F.Cu B.Cu) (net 20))
 (segment (start 186.1719 90.9219) (end 187.96 92.71) (width 0.75) (layer B.Cu) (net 20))
 (segment (start 132.9862 90.9219) (end 186.1719 90.9219) (width 0.75) (layer B.Cu) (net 20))
 (segment (start 132.2012 91.7069) (end 132.9862 90.9219) (width 0.75) (layer B.Cu) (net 20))
 (segment (start 124.5223 108.1786) (end 122.0655 110.6354) (width 0.75) (layer F.Cu) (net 20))
 (segment (start 124.5223 99.3858) (end 124.5223 108.1786) (width 0.75) (layer F.Cu) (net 20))
 (segment (start 132.2012 91.7069) (end 124.5223 99.3858) (width 0.75) (layer F.Cu) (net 20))
 (segment (start 125.7609 114.3309) (end 122.0655 110.6354) (width 0.75) (layer F.Cu) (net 20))
 (segment (start 125.7609 121.9509) (end 125.7609 114.3309) (width 0.75) (layer F.Cu) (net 20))
 (segment (start 129.54 125.73) (end 125.7609 121.9509) (width 0.75) (layer F.Cu) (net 20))
 (segment (start 122.0655 110.6354) (end 121.92 110.49) (width 0.75) (layer F.Cu) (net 20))
 (via (at 161.4609 95.712) (size 0.7) (layers F.Cu B.Cu) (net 21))
 (segment (start 132.08 125.73) (end 132.08 127.0311) (width 0.75) (layer F.Cu) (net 21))
 (segment (start 128.4022 127.2304) (end 132.08 127.2304) (width 0.75) (layer F.Cu) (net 21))
 (segment (start 124.0963 122.9245) (end 128.4022 127.2304) (width 0.75) (layer F.Cu) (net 21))
 (segment (start 124.0963 115.2063) (end 124.0963 122.9245) (width 0.75) (layer F.Cu) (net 21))
 (segment (start 121.92 113.03) (end 124.0963 115.2063) (width 0.75) (layer F.Cu) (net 21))
 (segment (start 132.08 127.2304) (end 132.08 127.0311) (width 0.75) (layer F.Cu) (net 21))
 (segment (start 158.6183 98.5546) (end 161.4609 95.712) (width 0.75) (layer F.Cu) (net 21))
 (segment (start 158.6183 107.2824) (end 158.6183 98.5546) (width 0.75) (layer F.Cu) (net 21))
 (segment (start 142.7015 123.1992) (end 158.6183 107.2824) (width 0.75) (layer F.Cu) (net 21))
 (segment (start 140.1791 123.1992) (end 142.7015 123.1992) (width 0.75) (layer F.Cu) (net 21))
 (segment (start 136.1479 127.2304) (end 140.1791 123.1992) (width 0.75) (layer F.Cu) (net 21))
 (segment (start 132.08 127.2304) (end 136.1479 127.2304) (width 0.75) (layer F.Cu) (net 21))
 (segment (start 182.7747 95.3553) (end 185.42 92.71) (width 0.75) (layer B.Cu) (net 21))
 (segment (start 161.8176 95.3553) (end 182.7747 95.3553) (width 0.75) (layer B.Cu) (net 21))
 (segment (start 161.4609 95.712) (end 161.8176 95.3553) (width 0.75) (layer B.Cu) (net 21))
 (segment (start 210.82 95.25) (end 210.82 85.09) (width 0.75) (layer F.Cu) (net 28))
 (segment (start 222.25 106.68) (end 210.82 95.25) (width 0.75) (layer F.Cu) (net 28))
 (segment (start 143.51 125.73) (end 145.276 125.73) (width 0.75) (layer B.Cu) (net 6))
 (segment (start 145.276 125.73) (end 152.896 118.11) (width 0.75) (layer B.Cu) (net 6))
 (segment (start 152.896 118.11) (end 203.2 118.11) (width 0.75) (layer B.Cu) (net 6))
 (segment (start 133.35 105.41) (end 134.75 105.41) (width 0.75) (layer B.Cu) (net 6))
 (segment (start 143.51 105.41) (end 134.75 105.41) (width 0.75) (layer B.Cu) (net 6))
 (segment (start 143.51 108.724) (end 143.51 105.41) (width 0.75) (layer B.Cu) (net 6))
 (segment (start 152.896 118.11) (end 143.51 108.724) (width 0.75) (layer B.Cu) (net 6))
 (segment (start 143.51 105.41) (end 143.51 105.1611) (width 0.75) (layer B.Cu) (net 6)))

